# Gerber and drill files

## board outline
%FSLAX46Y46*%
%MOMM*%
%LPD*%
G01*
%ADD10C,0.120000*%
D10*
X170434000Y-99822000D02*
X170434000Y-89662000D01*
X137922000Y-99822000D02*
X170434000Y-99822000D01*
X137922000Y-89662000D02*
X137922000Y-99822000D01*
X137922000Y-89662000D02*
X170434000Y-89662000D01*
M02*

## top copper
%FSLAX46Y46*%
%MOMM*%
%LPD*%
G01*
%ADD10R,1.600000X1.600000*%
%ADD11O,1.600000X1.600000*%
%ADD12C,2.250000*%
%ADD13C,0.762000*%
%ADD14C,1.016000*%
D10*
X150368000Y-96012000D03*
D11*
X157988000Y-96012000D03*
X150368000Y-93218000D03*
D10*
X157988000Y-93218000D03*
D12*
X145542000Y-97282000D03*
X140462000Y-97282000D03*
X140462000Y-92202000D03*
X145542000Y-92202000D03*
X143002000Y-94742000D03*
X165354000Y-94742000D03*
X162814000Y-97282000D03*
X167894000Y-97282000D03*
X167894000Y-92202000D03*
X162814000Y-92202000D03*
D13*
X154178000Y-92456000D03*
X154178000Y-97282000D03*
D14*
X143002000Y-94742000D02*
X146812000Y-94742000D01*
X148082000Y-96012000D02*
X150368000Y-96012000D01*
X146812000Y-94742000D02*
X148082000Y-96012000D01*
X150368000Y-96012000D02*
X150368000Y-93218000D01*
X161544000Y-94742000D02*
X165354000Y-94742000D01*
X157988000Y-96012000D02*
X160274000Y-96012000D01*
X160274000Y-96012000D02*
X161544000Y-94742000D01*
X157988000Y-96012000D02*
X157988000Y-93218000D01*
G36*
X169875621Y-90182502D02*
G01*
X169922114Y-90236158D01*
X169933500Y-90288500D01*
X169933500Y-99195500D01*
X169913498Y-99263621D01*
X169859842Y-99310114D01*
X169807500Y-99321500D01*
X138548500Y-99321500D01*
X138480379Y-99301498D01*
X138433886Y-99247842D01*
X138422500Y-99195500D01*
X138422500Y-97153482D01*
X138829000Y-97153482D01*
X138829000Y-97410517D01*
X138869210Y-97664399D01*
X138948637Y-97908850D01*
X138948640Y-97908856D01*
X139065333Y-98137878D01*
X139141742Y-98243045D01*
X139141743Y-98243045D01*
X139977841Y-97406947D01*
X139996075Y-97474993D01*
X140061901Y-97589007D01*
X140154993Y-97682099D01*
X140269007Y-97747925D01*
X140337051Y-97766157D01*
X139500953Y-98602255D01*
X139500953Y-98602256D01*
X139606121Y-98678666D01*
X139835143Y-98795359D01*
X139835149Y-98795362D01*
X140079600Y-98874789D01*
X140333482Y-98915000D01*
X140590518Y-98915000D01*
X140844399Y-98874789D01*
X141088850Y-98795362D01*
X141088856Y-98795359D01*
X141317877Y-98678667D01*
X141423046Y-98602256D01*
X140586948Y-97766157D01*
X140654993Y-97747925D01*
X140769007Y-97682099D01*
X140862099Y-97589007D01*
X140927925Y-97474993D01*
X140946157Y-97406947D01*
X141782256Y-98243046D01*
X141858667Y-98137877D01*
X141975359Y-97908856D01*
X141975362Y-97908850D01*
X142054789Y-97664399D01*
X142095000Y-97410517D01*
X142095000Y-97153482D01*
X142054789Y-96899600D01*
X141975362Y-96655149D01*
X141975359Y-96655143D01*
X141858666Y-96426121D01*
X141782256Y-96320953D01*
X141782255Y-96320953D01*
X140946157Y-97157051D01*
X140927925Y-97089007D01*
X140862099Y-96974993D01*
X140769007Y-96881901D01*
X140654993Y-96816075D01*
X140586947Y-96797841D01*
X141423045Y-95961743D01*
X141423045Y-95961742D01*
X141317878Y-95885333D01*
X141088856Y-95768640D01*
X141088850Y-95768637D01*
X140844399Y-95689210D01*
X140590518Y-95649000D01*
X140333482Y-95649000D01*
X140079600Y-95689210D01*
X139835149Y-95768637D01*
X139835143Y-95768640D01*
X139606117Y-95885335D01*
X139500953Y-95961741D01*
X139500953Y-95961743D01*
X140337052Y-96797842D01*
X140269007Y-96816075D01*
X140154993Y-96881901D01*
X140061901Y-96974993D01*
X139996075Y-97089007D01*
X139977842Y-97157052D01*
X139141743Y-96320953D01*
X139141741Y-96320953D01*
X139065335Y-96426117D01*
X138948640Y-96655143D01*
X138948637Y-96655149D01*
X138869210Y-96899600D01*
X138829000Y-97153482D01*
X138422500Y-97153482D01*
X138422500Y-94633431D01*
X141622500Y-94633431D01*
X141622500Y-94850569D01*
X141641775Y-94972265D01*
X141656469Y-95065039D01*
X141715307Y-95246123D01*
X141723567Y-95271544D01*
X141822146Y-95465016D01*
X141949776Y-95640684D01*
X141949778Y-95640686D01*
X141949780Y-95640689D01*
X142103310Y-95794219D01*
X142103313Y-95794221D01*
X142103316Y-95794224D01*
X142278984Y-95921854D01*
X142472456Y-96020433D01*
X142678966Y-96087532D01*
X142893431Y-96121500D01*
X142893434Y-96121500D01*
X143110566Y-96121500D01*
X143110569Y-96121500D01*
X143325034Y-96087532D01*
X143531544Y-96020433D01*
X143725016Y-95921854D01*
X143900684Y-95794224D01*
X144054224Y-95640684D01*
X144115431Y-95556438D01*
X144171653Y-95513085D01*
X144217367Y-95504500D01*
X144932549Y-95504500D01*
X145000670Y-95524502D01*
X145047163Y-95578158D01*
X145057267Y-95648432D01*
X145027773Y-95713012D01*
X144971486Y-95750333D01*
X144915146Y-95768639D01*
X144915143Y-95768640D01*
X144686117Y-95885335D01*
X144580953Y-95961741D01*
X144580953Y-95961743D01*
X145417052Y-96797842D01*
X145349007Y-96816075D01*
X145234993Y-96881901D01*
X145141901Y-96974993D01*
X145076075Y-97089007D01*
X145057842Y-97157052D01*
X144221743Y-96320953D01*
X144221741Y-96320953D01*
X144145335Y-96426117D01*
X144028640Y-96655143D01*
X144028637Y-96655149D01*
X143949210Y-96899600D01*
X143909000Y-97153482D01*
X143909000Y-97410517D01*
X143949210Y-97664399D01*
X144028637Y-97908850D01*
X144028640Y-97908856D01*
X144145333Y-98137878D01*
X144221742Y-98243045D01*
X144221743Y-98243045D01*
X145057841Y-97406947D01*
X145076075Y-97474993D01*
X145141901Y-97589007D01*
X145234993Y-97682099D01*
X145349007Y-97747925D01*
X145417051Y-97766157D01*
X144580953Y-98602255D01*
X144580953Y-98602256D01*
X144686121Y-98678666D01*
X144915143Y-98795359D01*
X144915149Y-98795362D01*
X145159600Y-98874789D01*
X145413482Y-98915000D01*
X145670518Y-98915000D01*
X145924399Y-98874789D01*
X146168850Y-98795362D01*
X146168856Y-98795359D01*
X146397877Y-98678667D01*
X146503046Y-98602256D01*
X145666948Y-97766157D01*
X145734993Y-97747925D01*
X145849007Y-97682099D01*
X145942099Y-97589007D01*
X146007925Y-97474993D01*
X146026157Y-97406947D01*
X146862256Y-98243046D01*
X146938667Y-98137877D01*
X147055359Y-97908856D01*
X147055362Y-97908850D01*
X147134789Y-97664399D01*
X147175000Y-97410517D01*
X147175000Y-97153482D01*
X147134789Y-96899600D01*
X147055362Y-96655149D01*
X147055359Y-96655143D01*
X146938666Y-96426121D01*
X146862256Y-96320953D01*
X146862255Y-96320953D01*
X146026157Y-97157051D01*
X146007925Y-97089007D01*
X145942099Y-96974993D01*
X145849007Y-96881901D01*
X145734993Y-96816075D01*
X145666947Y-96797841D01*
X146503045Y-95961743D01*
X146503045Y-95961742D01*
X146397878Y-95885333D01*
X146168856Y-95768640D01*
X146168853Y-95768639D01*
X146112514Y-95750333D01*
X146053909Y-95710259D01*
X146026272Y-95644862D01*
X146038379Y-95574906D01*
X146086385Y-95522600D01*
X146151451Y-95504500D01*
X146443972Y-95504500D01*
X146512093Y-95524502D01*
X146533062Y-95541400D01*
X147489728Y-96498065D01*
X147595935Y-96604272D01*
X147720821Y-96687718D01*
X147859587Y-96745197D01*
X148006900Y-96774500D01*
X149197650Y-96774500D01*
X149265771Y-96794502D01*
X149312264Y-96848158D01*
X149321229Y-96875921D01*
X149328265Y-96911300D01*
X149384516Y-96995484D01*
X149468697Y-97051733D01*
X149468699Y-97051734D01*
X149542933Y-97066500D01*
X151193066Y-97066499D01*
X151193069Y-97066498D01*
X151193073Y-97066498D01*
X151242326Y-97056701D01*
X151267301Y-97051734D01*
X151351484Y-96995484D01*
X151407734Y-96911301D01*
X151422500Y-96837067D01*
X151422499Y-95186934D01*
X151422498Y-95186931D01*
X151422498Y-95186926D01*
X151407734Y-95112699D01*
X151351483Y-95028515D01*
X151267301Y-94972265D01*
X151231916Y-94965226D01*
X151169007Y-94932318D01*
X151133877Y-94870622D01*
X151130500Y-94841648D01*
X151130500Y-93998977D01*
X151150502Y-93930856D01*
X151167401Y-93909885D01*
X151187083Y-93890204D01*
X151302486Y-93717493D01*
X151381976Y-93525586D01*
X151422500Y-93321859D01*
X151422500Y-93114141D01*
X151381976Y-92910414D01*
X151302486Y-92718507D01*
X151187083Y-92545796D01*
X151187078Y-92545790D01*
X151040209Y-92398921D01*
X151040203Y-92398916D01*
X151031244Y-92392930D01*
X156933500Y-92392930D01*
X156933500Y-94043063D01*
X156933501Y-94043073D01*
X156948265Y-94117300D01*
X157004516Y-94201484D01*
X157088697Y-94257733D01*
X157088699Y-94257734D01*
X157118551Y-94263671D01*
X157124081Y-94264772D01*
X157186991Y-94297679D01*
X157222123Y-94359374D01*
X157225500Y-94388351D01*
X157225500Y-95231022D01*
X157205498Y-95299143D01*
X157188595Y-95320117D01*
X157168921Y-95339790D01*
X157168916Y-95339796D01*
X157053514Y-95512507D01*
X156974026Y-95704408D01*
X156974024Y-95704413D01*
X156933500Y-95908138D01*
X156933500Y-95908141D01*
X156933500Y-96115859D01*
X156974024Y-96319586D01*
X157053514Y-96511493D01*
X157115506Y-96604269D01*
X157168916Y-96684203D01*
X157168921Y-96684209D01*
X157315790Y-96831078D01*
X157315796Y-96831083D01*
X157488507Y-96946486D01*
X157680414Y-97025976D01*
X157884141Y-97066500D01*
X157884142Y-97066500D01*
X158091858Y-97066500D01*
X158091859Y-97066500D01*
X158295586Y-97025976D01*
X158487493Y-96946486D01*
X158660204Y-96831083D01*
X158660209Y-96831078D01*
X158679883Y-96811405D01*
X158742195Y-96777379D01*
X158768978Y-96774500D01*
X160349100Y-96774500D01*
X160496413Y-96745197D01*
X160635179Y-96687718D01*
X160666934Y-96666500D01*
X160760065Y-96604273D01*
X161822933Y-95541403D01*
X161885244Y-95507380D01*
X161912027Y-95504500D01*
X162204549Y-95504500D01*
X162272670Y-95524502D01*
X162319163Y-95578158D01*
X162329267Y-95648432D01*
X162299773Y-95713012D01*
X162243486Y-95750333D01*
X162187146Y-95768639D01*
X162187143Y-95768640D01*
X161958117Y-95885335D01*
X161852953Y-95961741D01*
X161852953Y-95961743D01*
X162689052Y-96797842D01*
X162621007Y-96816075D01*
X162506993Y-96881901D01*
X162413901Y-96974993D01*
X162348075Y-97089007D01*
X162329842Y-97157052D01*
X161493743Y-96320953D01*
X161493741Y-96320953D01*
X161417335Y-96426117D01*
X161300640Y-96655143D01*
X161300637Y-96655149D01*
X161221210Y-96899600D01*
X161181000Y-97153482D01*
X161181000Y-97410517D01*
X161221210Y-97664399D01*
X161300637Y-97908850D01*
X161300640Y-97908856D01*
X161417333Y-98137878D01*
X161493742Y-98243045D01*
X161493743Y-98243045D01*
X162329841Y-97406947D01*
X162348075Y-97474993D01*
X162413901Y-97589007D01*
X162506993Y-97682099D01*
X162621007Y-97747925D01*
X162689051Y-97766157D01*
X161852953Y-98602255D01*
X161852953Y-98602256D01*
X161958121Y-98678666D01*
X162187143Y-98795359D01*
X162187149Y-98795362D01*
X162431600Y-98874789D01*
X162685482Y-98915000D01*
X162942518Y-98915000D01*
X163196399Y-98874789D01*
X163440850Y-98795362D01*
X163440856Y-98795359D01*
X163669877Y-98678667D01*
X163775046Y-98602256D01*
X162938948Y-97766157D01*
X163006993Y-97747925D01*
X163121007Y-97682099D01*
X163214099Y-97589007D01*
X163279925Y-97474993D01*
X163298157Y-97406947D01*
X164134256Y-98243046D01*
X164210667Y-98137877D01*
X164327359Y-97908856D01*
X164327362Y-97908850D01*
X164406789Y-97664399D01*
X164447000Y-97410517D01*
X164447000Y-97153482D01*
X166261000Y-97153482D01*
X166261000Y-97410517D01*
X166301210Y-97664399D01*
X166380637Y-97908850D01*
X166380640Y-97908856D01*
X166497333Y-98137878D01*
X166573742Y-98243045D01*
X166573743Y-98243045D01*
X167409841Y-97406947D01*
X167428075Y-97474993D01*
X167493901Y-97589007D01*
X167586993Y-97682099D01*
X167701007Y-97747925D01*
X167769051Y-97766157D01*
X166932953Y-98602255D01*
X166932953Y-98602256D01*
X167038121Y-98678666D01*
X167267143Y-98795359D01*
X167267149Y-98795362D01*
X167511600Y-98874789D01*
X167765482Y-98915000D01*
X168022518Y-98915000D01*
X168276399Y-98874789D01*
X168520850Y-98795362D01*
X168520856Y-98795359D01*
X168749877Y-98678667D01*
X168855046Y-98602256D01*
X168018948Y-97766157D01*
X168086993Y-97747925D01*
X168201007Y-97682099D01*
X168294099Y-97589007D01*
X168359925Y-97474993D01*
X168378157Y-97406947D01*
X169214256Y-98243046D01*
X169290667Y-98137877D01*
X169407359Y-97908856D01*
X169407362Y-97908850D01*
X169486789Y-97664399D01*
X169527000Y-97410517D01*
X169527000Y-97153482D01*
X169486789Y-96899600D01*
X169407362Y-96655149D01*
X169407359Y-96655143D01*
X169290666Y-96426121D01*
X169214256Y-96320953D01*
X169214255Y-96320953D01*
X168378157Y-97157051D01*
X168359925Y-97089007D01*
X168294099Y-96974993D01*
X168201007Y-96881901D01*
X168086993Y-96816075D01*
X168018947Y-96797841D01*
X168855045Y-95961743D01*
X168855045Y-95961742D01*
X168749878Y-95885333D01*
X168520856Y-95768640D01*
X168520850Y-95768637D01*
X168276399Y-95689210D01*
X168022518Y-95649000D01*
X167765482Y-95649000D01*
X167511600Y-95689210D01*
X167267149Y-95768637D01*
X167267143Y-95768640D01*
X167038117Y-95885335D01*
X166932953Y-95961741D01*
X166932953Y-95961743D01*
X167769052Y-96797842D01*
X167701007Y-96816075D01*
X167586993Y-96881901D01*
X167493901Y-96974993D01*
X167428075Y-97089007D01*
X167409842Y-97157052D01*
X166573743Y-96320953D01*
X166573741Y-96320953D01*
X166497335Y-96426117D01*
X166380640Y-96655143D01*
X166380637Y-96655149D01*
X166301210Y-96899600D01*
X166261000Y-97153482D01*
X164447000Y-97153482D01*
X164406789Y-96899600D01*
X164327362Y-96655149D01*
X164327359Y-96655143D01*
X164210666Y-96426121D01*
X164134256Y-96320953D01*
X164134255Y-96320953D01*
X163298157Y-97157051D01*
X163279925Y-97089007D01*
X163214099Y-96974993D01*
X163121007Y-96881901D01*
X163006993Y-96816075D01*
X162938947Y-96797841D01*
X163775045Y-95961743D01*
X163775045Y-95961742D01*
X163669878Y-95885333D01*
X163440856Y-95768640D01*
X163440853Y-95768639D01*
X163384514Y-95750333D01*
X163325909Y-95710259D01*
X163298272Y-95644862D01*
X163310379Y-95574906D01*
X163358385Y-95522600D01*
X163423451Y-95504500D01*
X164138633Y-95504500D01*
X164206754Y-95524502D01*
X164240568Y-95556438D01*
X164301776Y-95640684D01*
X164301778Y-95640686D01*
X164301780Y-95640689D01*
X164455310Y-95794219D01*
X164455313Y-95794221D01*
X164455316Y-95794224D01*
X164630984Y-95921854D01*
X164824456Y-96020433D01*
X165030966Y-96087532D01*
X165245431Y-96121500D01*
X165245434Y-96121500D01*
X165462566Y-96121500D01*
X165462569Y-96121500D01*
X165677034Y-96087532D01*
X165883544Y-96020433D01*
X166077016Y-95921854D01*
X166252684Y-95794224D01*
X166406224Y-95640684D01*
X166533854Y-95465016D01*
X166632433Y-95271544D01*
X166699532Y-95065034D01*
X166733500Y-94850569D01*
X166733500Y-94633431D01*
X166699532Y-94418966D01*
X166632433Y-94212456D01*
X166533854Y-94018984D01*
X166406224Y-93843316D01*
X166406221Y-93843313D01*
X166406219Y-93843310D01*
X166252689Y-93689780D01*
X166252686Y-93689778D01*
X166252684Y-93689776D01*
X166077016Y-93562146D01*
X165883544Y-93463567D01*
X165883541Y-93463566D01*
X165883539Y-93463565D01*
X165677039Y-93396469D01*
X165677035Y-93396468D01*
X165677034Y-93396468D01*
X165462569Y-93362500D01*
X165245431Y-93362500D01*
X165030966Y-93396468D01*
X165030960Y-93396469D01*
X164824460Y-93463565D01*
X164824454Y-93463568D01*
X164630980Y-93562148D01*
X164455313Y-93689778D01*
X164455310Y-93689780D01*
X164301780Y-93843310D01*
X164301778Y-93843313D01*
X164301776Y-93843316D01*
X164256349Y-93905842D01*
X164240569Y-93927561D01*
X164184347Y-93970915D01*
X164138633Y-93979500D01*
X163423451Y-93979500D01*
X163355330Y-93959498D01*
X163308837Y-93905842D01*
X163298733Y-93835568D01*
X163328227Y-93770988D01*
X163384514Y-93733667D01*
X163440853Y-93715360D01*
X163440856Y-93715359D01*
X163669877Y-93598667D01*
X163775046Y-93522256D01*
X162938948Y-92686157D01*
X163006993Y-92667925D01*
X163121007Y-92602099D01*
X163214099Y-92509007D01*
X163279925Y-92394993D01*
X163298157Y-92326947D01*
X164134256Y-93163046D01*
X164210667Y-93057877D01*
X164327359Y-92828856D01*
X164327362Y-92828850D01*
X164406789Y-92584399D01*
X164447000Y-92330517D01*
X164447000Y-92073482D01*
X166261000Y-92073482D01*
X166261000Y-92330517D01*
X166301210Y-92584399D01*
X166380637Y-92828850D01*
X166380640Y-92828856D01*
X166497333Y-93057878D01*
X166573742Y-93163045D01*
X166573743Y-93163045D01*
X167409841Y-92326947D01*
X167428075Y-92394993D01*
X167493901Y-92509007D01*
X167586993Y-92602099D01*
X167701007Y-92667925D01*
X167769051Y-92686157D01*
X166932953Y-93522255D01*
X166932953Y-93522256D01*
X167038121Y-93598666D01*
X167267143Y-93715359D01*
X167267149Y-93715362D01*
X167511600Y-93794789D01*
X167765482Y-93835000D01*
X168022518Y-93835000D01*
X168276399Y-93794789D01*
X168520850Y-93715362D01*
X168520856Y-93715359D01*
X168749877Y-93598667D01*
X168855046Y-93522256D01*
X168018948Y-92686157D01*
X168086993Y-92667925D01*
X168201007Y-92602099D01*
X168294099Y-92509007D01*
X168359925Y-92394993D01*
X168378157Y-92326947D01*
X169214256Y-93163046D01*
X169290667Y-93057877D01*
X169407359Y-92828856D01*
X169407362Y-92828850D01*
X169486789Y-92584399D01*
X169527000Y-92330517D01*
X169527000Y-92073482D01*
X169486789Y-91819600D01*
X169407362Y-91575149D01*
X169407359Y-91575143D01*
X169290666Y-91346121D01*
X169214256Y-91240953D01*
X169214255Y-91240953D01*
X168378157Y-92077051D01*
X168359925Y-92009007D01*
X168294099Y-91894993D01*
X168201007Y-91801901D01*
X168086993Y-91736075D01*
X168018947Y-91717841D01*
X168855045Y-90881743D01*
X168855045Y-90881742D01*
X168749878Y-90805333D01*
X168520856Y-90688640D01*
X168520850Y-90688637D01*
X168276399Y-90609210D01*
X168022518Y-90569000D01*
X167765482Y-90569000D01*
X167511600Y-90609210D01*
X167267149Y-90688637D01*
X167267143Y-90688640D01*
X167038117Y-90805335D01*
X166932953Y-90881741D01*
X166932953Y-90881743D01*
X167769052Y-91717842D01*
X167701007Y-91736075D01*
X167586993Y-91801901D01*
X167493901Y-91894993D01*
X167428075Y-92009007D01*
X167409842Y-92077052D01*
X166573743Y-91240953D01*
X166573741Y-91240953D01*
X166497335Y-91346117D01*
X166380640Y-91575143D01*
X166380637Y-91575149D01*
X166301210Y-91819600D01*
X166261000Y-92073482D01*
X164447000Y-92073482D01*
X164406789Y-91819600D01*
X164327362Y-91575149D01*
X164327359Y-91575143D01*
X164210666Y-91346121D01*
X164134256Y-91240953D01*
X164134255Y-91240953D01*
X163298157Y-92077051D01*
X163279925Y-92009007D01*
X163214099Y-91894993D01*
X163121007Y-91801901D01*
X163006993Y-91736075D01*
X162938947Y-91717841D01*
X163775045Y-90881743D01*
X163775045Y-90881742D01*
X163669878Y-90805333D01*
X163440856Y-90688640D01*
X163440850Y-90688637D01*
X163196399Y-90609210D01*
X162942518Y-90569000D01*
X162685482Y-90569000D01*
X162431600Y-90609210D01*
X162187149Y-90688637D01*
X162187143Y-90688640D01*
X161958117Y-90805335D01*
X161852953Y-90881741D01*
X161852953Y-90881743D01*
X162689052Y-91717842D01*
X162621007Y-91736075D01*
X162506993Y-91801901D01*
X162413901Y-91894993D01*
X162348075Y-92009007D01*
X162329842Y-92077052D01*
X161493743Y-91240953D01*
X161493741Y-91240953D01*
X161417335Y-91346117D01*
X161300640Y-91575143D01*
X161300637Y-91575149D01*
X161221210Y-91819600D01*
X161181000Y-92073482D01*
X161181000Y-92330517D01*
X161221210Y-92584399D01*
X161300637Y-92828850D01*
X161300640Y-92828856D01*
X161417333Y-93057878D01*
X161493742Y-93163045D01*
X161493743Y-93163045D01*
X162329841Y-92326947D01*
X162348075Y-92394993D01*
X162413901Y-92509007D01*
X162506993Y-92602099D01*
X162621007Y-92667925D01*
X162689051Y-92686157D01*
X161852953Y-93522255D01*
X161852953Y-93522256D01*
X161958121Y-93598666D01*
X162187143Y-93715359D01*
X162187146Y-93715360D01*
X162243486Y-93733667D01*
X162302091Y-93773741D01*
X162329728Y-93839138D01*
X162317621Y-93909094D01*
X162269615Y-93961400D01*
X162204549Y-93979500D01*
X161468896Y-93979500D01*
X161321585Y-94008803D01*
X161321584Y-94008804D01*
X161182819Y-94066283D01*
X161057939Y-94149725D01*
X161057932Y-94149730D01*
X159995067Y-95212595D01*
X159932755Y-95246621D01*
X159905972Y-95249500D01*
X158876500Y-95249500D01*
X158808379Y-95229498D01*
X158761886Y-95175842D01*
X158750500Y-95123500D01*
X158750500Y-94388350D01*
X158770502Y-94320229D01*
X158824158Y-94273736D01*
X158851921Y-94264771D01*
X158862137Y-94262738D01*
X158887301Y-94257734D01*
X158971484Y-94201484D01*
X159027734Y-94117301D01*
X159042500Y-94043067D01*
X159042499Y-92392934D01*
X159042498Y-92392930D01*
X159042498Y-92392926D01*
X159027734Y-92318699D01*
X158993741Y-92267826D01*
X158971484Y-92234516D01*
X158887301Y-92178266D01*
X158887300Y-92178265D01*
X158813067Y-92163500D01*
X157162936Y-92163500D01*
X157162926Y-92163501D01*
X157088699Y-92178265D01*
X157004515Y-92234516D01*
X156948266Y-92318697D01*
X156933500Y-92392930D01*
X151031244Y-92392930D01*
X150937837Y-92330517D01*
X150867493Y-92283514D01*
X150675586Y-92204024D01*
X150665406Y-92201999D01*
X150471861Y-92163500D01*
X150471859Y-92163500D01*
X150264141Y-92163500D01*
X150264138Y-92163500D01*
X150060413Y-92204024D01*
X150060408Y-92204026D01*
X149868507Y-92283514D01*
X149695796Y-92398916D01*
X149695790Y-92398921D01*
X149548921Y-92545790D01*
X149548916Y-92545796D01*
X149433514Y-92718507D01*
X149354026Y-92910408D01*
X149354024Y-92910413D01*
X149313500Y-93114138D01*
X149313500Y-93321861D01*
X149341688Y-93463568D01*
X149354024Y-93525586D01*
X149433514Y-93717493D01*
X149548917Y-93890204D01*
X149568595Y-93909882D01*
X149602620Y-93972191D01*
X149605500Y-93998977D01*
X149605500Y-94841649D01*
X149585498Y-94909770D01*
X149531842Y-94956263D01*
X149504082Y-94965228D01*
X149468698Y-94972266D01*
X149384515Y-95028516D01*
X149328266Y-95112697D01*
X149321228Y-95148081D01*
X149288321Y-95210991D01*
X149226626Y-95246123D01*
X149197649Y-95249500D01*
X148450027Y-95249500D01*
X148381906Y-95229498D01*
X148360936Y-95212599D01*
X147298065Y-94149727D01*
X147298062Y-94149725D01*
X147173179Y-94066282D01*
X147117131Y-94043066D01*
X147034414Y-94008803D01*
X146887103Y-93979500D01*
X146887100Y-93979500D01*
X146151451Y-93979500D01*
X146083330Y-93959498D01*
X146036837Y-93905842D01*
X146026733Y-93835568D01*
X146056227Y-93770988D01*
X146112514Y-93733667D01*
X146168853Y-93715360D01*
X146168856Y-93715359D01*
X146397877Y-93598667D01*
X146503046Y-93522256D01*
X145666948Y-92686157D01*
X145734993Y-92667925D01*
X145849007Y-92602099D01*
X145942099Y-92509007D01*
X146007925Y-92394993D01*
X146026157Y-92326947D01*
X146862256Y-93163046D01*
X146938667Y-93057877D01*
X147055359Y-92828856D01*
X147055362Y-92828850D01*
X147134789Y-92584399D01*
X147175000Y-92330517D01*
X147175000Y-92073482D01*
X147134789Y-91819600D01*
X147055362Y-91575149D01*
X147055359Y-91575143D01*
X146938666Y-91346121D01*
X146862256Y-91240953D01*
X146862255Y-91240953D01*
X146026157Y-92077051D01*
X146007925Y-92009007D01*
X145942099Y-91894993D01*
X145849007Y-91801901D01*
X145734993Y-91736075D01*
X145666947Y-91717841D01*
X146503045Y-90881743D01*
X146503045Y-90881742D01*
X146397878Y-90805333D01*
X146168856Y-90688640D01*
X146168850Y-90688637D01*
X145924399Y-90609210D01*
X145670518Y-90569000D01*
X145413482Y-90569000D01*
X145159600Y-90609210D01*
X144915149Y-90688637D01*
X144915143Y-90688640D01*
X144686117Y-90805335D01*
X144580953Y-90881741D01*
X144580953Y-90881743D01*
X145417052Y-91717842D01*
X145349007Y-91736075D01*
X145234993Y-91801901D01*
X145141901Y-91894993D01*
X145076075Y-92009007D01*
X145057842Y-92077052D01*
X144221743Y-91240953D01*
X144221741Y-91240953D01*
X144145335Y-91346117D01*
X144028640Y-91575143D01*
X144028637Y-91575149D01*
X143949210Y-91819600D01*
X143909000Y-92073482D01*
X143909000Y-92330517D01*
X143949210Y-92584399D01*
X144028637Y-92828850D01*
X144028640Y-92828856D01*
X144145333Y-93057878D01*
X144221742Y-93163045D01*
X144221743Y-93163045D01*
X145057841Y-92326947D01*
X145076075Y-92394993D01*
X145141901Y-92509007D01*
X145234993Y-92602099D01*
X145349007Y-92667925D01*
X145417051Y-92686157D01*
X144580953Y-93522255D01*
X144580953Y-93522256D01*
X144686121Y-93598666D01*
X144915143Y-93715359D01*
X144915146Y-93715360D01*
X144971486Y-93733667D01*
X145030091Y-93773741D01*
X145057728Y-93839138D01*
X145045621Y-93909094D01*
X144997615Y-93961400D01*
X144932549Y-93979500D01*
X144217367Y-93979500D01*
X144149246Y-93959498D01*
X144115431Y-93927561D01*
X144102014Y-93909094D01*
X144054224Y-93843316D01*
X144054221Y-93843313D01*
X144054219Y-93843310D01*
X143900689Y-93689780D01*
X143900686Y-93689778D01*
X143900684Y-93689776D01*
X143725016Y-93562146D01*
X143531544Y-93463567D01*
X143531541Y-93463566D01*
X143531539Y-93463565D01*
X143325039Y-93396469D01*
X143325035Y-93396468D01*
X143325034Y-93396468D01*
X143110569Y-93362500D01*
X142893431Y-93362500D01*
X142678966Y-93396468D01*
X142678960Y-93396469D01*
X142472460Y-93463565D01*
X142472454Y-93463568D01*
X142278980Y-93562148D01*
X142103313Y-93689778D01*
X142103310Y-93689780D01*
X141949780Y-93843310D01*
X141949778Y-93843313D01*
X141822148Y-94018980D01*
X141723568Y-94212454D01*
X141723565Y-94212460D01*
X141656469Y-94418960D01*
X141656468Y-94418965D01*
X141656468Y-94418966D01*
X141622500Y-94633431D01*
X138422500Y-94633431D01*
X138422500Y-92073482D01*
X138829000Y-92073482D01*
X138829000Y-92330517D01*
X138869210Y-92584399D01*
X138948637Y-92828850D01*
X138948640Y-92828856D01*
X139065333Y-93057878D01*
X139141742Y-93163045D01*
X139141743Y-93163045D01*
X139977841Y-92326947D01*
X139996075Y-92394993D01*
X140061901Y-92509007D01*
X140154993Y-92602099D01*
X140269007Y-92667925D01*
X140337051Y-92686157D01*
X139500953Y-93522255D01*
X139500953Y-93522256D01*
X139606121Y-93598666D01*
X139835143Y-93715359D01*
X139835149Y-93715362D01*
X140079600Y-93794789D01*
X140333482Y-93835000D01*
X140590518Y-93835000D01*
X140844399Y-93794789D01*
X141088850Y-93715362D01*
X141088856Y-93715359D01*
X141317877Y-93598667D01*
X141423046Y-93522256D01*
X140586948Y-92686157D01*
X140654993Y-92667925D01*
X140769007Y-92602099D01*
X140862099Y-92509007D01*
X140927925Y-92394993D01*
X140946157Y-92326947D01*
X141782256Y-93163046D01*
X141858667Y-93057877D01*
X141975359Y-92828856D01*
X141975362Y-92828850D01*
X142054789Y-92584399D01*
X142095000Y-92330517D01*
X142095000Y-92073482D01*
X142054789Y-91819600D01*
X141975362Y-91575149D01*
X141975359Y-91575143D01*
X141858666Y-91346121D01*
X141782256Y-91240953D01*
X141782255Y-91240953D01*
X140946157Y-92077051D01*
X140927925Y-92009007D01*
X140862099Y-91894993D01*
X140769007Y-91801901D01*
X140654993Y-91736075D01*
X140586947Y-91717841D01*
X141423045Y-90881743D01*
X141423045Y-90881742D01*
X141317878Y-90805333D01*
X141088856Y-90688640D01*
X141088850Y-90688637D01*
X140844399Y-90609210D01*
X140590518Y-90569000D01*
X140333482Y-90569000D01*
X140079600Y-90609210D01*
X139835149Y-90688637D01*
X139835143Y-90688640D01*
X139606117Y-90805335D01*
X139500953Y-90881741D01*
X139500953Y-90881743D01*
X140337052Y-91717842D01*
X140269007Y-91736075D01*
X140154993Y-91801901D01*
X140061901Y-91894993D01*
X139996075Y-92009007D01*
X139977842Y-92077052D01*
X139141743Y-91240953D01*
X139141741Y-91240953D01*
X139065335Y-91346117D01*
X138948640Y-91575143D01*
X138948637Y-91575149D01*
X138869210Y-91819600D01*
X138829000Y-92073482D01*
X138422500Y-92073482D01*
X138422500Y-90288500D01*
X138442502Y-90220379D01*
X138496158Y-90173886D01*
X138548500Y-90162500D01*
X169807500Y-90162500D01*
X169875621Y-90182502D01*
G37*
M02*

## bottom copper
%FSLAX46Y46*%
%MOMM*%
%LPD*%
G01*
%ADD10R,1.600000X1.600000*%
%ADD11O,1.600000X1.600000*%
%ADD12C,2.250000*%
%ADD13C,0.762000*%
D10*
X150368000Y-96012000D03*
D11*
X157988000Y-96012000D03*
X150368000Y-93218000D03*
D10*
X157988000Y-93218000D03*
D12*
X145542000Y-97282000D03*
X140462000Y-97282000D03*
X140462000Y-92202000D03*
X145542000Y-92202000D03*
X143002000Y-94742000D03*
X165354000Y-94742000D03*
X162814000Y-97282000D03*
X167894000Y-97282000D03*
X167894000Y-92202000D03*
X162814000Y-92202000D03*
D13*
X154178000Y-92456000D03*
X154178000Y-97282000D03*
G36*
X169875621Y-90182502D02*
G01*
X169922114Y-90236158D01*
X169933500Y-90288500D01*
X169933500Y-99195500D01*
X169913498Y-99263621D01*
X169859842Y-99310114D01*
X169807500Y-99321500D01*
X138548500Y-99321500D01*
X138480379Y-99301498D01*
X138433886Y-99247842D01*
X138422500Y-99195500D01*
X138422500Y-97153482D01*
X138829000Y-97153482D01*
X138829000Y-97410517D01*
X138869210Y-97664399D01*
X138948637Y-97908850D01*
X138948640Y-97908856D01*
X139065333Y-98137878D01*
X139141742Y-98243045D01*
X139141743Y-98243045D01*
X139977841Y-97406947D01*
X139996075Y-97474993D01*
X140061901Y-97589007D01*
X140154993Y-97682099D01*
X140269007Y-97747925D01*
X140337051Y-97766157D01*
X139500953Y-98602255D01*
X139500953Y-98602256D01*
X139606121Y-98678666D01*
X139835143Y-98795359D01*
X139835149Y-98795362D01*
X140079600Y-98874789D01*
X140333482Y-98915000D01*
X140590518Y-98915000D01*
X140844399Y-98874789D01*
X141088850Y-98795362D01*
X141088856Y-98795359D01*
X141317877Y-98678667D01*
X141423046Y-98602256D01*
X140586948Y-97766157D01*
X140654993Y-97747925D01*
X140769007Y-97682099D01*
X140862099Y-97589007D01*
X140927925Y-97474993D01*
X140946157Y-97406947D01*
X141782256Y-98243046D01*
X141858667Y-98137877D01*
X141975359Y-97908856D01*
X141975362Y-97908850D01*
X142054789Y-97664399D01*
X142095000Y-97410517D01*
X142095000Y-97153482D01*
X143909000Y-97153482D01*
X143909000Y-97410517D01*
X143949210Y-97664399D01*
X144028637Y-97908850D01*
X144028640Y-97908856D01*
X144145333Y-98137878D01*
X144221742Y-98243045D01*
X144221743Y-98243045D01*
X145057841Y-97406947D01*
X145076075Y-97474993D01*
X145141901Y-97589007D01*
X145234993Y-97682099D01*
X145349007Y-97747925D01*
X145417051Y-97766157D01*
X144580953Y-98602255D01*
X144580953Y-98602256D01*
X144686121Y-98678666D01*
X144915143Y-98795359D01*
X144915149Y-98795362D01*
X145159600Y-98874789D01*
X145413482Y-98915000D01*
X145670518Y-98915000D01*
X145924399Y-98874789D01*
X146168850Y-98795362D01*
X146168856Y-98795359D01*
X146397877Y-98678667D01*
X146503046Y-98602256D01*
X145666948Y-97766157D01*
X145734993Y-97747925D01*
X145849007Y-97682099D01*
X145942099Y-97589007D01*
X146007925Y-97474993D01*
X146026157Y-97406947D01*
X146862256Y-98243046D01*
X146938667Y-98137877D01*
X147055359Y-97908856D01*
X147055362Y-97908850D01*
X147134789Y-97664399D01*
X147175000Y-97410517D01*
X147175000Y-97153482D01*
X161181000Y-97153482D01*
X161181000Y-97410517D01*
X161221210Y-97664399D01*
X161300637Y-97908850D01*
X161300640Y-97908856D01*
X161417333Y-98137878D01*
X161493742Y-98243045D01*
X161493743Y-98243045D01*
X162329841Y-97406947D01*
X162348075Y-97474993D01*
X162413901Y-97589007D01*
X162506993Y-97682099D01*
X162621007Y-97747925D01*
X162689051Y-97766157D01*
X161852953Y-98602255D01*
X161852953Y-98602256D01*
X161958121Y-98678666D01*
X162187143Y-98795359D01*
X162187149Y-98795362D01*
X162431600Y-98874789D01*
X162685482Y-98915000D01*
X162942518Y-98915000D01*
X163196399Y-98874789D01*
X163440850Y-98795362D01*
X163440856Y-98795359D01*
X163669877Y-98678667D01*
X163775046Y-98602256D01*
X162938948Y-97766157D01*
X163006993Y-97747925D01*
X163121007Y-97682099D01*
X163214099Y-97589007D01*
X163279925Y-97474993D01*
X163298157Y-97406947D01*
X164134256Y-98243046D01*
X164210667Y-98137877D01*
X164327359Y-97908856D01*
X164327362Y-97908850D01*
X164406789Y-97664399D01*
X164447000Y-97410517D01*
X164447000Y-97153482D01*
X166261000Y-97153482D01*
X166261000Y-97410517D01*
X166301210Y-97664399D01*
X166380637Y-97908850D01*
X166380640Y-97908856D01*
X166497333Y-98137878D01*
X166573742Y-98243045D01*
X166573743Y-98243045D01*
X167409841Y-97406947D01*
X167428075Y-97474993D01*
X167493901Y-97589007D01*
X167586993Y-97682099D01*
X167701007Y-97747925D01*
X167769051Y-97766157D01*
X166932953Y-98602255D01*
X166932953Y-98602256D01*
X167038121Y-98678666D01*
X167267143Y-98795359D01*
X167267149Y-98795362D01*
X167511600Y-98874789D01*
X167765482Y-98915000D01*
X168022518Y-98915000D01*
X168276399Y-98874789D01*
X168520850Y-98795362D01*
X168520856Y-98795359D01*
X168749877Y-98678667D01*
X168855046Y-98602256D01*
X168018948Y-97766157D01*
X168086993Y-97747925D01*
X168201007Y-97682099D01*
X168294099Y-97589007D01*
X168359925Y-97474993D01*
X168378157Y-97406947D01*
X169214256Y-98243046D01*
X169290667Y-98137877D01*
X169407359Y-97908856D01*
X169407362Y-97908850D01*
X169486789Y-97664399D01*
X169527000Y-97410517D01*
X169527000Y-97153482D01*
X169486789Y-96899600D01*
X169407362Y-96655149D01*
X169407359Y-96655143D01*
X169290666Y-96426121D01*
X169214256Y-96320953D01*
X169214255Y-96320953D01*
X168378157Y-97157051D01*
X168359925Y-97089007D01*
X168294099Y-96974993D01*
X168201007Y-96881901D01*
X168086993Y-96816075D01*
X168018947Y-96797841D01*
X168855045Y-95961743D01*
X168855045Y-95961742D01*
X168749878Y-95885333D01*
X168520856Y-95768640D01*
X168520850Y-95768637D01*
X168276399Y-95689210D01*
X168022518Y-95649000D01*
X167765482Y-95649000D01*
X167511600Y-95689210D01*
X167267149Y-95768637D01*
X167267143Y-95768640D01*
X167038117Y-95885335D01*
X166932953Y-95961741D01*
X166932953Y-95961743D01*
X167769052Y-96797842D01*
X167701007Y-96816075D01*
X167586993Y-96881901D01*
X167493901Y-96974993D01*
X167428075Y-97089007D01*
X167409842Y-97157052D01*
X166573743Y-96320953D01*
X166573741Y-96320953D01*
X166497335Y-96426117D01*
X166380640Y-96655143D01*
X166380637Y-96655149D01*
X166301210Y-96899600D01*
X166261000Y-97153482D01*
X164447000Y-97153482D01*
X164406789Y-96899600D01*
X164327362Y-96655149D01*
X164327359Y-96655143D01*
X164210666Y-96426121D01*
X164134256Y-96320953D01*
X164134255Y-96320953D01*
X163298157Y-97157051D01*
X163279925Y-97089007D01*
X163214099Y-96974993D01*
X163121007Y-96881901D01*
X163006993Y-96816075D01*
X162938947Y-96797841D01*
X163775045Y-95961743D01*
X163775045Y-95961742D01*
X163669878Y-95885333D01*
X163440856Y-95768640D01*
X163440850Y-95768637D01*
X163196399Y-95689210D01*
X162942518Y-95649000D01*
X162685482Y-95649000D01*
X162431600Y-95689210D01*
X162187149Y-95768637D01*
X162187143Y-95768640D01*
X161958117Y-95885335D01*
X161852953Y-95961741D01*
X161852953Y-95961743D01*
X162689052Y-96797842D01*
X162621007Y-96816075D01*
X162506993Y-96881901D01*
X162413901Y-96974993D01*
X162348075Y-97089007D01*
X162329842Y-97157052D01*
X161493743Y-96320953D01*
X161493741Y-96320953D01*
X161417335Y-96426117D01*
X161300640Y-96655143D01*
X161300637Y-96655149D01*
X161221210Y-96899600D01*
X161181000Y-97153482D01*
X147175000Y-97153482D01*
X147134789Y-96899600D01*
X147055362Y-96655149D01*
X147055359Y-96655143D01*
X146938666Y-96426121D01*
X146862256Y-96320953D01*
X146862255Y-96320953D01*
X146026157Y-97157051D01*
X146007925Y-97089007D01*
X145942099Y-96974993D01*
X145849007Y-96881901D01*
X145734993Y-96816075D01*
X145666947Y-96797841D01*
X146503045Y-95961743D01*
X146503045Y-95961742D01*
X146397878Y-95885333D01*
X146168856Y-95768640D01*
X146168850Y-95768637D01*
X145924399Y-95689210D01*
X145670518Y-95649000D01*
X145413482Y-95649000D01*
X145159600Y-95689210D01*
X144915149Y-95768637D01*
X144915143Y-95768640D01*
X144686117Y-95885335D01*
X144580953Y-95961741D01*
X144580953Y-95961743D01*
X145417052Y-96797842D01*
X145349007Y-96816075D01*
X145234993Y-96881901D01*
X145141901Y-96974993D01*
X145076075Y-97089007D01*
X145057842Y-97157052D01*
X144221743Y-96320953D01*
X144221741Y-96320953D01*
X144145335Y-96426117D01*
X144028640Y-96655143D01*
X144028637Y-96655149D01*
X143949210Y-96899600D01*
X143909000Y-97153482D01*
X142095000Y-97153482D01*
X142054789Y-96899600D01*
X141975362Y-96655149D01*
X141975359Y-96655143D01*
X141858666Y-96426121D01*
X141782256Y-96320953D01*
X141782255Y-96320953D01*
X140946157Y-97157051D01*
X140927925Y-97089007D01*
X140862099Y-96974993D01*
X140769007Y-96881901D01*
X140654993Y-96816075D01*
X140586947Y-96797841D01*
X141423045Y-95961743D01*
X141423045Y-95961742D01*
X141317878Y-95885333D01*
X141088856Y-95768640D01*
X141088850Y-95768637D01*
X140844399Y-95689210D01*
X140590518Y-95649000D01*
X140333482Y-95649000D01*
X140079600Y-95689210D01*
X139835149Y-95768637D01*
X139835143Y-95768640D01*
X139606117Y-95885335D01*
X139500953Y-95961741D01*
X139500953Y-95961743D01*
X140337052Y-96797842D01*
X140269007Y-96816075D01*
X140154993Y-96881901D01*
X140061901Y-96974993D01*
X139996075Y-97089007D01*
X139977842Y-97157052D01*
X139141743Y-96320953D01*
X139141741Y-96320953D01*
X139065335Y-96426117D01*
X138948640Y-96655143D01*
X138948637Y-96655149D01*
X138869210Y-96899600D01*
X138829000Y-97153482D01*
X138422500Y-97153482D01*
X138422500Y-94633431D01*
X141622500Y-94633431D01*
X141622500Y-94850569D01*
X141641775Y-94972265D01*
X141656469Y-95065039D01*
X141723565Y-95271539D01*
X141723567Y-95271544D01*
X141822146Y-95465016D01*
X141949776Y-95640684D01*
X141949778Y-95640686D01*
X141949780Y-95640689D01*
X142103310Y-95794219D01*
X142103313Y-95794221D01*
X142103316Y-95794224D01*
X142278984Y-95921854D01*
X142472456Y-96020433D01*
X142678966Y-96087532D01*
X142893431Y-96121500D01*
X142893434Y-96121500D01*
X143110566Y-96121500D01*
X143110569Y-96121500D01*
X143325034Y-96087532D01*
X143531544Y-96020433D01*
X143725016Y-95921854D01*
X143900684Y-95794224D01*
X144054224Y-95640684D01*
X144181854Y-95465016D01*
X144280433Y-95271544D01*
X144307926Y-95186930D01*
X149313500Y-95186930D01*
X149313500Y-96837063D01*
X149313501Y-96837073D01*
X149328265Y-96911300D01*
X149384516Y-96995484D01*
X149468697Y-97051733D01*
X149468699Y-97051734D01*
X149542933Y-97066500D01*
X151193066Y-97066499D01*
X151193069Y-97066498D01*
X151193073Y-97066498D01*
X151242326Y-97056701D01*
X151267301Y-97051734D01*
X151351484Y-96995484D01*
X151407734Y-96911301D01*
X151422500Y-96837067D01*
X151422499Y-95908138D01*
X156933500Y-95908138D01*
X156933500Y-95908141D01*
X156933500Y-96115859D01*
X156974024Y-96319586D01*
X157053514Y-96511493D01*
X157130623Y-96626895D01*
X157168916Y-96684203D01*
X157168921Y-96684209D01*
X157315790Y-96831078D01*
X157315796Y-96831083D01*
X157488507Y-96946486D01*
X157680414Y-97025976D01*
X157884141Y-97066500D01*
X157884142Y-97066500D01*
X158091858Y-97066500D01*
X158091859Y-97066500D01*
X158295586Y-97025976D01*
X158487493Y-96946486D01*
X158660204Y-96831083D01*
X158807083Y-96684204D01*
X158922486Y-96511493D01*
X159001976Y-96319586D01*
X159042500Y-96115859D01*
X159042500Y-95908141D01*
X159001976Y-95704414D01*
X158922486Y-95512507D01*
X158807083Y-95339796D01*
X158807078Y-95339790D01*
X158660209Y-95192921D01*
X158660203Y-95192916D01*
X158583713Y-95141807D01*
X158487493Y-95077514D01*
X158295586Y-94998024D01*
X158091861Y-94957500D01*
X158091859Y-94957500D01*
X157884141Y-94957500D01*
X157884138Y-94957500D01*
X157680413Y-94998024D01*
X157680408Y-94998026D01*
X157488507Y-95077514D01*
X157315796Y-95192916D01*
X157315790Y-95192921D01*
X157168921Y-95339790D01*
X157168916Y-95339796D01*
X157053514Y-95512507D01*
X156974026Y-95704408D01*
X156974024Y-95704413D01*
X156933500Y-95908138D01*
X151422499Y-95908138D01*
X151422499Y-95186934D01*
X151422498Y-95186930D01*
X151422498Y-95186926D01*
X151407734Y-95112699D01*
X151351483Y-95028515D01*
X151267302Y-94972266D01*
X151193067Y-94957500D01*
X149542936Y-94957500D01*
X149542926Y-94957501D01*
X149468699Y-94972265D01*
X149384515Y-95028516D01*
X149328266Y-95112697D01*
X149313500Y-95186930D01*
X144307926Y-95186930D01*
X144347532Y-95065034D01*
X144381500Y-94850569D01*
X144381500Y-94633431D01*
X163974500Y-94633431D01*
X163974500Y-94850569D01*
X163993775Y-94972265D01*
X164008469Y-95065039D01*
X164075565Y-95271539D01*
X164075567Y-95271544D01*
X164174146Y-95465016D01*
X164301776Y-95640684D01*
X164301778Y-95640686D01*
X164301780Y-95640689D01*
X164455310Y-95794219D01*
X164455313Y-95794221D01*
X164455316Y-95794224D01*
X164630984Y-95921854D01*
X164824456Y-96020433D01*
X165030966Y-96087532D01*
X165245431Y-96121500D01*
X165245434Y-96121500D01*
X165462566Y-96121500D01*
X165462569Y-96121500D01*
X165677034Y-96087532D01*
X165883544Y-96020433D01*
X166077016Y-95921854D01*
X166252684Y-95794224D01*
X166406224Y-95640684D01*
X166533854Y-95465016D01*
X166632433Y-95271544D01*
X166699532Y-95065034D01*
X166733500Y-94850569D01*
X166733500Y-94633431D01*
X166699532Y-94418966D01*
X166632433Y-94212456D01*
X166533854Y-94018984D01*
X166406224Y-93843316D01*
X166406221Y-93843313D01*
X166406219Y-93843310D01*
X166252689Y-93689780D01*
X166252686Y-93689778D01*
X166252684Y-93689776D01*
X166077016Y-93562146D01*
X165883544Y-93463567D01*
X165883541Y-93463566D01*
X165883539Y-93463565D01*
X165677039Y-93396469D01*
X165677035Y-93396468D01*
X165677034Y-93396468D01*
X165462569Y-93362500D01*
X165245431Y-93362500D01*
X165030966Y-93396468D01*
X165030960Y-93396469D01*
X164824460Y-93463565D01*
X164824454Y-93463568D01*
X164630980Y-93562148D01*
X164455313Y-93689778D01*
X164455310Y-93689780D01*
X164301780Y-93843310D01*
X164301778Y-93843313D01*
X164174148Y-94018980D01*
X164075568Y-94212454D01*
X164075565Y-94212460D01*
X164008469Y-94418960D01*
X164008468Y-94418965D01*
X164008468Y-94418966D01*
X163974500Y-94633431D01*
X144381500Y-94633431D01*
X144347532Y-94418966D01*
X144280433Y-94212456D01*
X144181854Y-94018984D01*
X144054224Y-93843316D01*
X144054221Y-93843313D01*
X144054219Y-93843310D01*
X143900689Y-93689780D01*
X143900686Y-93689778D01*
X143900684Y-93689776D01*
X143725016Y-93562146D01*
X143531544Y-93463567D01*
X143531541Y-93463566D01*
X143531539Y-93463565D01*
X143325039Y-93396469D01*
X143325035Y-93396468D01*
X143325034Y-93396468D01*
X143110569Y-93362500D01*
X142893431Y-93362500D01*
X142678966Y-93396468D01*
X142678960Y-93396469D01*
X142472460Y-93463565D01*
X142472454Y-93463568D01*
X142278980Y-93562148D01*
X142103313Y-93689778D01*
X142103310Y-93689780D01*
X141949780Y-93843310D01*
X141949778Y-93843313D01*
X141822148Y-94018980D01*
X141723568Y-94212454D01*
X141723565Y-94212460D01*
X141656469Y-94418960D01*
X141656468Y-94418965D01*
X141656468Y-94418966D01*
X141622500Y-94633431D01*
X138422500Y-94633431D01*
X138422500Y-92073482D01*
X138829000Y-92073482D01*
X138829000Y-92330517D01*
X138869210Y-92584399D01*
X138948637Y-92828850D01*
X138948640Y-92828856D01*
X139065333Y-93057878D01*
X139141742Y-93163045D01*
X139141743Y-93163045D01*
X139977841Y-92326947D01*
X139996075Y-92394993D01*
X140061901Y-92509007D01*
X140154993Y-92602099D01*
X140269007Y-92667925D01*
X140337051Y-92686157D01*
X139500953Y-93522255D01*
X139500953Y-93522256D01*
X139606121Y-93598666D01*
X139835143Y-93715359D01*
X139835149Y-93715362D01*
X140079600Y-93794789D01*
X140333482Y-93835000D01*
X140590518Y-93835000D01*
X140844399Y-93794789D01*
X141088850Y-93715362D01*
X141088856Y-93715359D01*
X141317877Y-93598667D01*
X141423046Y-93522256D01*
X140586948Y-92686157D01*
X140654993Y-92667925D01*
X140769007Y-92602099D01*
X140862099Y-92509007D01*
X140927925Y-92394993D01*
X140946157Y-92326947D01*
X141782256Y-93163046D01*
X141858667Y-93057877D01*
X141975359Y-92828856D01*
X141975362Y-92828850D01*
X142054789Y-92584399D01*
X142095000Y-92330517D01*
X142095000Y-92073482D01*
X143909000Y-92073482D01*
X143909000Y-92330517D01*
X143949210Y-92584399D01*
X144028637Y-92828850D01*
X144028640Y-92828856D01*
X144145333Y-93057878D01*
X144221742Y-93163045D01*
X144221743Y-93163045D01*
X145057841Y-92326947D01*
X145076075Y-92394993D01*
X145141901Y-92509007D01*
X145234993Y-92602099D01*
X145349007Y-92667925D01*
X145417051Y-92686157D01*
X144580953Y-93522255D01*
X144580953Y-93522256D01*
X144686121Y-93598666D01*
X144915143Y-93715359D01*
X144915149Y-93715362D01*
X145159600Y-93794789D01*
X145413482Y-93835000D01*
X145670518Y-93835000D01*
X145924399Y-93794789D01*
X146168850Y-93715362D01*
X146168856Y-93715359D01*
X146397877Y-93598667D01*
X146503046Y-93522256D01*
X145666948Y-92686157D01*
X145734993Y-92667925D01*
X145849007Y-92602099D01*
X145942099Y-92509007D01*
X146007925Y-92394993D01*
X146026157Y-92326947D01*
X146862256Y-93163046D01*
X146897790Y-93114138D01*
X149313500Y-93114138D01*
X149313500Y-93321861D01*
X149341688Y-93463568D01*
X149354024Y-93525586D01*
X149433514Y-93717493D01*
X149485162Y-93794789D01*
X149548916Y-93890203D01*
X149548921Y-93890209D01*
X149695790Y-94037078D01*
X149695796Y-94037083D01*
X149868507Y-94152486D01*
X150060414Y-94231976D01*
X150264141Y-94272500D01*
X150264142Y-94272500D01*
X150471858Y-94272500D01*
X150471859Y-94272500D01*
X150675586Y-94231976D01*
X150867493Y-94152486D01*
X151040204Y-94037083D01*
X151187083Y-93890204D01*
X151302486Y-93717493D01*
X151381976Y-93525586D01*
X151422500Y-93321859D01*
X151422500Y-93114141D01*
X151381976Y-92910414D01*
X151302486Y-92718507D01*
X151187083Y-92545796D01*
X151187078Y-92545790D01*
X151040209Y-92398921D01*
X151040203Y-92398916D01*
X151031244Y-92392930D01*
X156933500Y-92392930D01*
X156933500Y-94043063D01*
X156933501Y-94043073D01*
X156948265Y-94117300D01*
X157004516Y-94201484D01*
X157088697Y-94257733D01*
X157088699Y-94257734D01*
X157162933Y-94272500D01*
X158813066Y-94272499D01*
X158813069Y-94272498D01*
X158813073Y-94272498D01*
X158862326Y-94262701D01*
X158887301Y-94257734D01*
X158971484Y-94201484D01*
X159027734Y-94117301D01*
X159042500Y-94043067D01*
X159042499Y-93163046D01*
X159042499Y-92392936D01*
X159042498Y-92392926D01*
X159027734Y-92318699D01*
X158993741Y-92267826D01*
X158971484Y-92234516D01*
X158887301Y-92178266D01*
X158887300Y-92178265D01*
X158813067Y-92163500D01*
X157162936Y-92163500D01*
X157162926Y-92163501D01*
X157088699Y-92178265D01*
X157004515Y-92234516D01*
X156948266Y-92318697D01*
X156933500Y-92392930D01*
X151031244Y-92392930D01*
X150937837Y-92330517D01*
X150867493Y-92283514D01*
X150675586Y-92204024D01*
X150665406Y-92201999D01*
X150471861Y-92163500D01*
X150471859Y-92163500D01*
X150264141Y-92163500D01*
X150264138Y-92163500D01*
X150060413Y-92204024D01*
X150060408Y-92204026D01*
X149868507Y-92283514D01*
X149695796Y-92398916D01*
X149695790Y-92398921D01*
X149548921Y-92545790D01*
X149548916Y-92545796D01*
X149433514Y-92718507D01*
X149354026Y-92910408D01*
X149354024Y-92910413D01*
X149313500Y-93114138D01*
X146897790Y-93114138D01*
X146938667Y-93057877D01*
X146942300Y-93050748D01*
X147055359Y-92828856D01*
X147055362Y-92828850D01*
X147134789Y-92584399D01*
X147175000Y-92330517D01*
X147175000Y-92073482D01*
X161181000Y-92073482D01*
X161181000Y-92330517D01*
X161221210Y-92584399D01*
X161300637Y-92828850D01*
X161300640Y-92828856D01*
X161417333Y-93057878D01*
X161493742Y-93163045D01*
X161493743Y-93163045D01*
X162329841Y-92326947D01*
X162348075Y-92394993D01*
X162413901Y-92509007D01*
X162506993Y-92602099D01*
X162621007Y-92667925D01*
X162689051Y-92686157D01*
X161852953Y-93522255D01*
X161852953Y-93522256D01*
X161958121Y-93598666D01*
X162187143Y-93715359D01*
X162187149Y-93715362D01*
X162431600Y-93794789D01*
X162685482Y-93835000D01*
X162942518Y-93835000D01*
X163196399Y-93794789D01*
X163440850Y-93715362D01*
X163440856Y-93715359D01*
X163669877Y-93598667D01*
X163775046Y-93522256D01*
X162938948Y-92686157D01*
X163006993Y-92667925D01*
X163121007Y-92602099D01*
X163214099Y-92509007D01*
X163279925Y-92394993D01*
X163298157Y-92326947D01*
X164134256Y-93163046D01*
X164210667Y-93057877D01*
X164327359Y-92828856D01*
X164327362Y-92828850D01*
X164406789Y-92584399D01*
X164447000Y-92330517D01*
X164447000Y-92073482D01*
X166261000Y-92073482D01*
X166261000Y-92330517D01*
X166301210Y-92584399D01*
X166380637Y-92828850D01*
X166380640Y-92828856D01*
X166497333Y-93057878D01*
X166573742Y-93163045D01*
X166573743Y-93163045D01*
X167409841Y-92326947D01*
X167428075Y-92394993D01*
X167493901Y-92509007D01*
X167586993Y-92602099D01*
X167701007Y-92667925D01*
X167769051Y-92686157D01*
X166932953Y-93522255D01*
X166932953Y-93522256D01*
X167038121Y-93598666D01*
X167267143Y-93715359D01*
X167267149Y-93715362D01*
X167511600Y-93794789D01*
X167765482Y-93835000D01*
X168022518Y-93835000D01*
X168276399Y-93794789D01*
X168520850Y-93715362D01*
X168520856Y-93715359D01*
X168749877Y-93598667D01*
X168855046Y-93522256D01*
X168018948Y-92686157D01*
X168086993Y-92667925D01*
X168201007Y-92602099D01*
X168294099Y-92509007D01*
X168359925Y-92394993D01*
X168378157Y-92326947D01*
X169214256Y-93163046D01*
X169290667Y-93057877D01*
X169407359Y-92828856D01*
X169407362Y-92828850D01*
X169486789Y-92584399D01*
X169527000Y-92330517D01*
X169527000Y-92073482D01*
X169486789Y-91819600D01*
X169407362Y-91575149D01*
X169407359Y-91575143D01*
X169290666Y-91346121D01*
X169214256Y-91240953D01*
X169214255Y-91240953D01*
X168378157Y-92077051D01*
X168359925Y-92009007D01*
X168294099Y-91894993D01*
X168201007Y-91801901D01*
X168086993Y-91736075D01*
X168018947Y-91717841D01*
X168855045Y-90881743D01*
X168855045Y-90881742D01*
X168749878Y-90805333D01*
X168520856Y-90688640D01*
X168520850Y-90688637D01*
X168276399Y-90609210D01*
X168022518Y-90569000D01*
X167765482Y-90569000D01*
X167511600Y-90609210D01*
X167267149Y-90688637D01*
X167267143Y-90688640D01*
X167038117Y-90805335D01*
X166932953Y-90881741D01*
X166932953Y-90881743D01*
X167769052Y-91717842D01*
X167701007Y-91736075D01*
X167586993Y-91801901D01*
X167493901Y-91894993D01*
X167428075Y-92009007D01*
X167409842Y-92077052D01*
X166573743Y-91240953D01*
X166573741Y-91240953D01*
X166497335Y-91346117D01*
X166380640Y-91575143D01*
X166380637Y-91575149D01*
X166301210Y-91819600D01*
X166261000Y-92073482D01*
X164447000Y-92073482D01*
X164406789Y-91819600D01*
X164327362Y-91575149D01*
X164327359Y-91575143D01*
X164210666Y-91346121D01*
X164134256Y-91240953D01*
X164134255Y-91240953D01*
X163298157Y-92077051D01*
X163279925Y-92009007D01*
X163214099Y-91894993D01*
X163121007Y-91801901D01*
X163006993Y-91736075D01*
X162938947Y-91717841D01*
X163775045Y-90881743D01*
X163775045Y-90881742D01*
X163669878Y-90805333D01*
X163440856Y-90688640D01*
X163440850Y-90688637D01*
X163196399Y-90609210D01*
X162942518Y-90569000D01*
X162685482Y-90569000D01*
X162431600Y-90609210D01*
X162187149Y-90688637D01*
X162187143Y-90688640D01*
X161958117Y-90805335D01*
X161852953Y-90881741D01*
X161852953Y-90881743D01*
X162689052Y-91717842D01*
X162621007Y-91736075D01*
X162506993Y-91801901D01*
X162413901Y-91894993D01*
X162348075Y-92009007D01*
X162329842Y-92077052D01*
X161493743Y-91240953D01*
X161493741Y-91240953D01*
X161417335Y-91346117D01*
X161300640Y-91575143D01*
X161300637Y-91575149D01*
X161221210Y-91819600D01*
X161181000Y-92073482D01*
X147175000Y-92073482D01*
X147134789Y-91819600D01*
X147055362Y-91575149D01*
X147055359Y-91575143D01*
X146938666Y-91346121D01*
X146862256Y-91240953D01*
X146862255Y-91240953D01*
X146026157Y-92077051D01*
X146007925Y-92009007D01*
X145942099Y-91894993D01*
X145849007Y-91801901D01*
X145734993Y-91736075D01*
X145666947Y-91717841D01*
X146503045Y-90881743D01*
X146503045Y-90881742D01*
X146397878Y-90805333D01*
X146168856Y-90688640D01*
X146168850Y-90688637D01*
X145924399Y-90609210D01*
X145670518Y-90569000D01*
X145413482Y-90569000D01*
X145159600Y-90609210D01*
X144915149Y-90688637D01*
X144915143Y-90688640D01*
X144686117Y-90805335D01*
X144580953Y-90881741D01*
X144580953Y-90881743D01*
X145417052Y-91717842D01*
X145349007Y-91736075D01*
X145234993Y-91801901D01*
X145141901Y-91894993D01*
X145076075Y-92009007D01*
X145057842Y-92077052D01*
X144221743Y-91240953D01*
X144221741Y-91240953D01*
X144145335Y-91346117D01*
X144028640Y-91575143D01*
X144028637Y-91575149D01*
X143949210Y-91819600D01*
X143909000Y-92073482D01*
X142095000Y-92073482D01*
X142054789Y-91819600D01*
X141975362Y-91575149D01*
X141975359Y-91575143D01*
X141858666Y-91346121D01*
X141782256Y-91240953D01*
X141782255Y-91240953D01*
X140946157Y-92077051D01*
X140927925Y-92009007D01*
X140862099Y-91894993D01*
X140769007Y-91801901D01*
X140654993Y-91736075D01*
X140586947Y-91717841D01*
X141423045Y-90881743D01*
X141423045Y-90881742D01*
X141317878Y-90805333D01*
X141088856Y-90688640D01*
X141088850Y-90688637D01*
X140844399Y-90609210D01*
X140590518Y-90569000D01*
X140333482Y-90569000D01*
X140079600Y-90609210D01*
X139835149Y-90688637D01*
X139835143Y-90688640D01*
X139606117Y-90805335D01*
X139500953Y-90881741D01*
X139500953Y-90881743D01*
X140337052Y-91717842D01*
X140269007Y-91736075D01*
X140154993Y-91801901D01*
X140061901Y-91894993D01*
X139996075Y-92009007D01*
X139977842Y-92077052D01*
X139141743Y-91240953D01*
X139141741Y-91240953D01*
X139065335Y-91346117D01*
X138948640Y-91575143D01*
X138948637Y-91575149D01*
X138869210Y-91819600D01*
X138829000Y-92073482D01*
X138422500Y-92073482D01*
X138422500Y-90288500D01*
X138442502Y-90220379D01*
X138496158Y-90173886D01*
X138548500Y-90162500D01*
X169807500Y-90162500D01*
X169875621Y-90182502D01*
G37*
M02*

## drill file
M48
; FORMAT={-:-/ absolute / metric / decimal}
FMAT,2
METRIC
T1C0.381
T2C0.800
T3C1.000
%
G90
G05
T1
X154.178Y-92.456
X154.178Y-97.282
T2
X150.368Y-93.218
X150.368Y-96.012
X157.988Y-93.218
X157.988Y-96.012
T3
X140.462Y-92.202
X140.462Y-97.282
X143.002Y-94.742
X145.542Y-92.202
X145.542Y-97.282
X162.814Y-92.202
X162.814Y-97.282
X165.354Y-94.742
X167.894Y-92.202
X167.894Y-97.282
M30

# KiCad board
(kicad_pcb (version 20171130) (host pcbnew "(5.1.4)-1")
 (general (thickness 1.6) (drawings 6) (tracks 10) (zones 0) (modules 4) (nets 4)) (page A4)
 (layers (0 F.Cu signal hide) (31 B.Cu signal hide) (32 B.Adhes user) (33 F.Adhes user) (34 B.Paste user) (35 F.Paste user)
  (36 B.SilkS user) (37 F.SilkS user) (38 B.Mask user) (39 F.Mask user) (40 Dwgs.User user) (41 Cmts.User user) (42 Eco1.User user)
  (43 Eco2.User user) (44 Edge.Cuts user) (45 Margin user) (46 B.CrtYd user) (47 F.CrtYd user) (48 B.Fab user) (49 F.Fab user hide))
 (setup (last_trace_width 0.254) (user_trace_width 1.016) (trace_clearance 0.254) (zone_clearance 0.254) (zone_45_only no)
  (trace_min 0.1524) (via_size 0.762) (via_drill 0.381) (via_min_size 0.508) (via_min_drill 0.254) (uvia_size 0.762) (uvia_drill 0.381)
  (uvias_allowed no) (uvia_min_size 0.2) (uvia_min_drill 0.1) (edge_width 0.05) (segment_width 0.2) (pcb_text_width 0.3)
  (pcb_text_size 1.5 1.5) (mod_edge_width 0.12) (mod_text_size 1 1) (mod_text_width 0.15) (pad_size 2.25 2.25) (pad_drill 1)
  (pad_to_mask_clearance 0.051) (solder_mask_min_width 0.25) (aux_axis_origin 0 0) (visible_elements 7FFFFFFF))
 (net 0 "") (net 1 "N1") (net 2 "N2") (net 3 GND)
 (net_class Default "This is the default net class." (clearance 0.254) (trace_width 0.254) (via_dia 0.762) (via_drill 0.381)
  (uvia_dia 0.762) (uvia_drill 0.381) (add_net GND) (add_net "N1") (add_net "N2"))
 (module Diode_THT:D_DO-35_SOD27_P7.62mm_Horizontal (layer F.Cu) (at 150.368 96.012)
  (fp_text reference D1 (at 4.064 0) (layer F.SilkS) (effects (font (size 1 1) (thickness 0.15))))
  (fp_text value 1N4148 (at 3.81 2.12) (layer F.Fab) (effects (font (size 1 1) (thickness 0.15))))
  (pad 1 thru_hole rect (at 0 0) (size 1.6 1.6) (drill 0.8) (layers *.Cu *.Mask) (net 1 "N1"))
  (pad 2 thru_hole oval (at 7.62 0) (size 1.6 1.6) (drill 0.8) (layers *.Cu *.Mask) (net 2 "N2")))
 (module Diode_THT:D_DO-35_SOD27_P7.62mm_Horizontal (layer F.Cu) (at 157.988 93.218 180)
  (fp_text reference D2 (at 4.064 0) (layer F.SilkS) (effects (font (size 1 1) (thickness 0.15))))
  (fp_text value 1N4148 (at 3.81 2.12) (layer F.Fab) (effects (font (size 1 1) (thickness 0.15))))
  (pad 2 thru_hole oval (at 7.62 0 180) (size 1.6 1.6) (drill 0.8) (layers *.Cu *.Mask) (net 1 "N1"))
  (pad 1 thru_hole rect (at 0 0 180) (size 1.6 1.6) (drill 0.8) (layers *.Cu *.Mask) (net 2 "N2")))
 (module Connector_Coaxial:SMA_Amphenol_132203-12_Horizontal (layer F.Cu) (at 143.002 94.742 90)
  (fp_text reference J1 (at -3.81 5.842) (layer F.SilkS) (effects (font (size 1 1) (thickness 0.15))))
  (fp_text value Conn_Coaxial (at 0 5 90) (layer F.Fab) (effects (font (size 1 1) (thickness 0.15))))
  (pad 2 thru_hole circle (at -2.54 2.54 90) (size 2.25 2.25) (drill 1) (layers *.Cu *.Mask) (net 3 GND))
  (pad 2 thru_hole circle (at -2.54 -2.54 90) (size 2.25 2.25) (drill 1) (layers *.Cu *.Mask) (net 3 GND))
  (pad 2 thru_hole circle (at 2.54 -2.54 90) (size 2.25 2.25) (drill 1) (layers *.Cu *.Mask) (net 3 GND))
  (pad 2 thru_hole circle (at 2.54 2.54 180) (size 2.25 2.25) (drill 1) (layers *.Cu *.Mask) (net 3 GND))
  (pad 1 thru_hole circle (at 0 0 90) (size 2.25 2.25) (drill 1) (layers *.Cu *.Mask) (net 1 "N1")))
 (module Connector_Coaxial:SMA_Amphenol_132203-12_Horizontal (layer F.Cu) (at 165.354 94.742 270)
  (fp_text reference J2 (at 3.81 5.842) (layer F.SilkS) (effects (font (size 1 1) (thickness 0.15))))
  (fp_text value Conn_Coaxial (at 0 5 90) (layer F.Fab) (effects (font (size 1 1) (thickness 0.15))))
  (pad 1 thru_hole circle (at 0 0 270) (size 2.25 2.25) (drill 1) (layers *.Cu *.Mask) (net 2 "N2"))
  (pad 2 thru_hole circle (at 2.54 2.54) (size 2.25 2.25) (drill 1) (layers *.Cu *.Mask) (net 3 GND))
  (pad 2 thru_hole circle (at 2.54 -2.54 270) (size 2.25 2.25) (drill 1) (layers *.Cu *.Mask) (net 3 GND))
  (pad 2 thru_hole circle (at -2.54 -2.54 270) (size 2.25 2.25) (drill 1) (layers *.Cu *.Mask) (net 3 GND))
  (pad 2 thru_hole circle (at -2.54 2.54 270) (size 2.25 2.25) (drill 1) (layers *.Cu *.Mask) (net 3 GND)))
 (gr_line (start 170.434 99.822) (end 170.434 89.662) (layer Edge.Cuts) (width 0.12))
 (gr_line (start 137.922 99.822) (end 170.434 99.822) (layer Edge.Cuts) (width 0.12))
 (gr_line (start 137.922 89.662) (end 137.922 99.822) (layer Edge.Cuts) (width 0.12))
 (gr_line (start 137.922 89.662) (end 170.434 89.662) (layer Edge.Cuts) (width 0.12))
 (segment (start 143.002 94.742) (end 146.812 94.742) (width 1.016) (layer F.Cu) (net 1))
 (segment (start 148.082 96.012) (end 150.368 96.012) (width 1.016) (layer F.Cu) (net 1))
 (segment (start 146.812 94.742) (end 148.082 96.012) (width 1.016) (layer F.Cu) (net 1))
 (segment (start 150.368 96.012) (end 150.368 93.218) (width 1.016) (layer F.Cu) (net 1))
 (segment (start 161.544 94.742) (end 165.354 94.742) (width 1.016) (layer F.Cu) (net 2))
 (segment (start 157.988 96.012) (end 160.274 96.012) (width 1.016) (layer F.Cu) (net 2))
 (segment (start 160.274 96.012) (end 161.544 94.742) (width 1.016) (layer F.Cu) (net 2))
 (segment (start 157.988 96.012) (end 157.988 93.218) (width 1.016) (layer F.Cu) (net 2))
 (via (at 154.178 92.456) (size 0.762) (drill 0.381) (layers F.Cu B.Cu) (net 3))
 (via (at 154.178 97.282) (size 0.762) (drill 0.381) (layers F.Cu B.Cu) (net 3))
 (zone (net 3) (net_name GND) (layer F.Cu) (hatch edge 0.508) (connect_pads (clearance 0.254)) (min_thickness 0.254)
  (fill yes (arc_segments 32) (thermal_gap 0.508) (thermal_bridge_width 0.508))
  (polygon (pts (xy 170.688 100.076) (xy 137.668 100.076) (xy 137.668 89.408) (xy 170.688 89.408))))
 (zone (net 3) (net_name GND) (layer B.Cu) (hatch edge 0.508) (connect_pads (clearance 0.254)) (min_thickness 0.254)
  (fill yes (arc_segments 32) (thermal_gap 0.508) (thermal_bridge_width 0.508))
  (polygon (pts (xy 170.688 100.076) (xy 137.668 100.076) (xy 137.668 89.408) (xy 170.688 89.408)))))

